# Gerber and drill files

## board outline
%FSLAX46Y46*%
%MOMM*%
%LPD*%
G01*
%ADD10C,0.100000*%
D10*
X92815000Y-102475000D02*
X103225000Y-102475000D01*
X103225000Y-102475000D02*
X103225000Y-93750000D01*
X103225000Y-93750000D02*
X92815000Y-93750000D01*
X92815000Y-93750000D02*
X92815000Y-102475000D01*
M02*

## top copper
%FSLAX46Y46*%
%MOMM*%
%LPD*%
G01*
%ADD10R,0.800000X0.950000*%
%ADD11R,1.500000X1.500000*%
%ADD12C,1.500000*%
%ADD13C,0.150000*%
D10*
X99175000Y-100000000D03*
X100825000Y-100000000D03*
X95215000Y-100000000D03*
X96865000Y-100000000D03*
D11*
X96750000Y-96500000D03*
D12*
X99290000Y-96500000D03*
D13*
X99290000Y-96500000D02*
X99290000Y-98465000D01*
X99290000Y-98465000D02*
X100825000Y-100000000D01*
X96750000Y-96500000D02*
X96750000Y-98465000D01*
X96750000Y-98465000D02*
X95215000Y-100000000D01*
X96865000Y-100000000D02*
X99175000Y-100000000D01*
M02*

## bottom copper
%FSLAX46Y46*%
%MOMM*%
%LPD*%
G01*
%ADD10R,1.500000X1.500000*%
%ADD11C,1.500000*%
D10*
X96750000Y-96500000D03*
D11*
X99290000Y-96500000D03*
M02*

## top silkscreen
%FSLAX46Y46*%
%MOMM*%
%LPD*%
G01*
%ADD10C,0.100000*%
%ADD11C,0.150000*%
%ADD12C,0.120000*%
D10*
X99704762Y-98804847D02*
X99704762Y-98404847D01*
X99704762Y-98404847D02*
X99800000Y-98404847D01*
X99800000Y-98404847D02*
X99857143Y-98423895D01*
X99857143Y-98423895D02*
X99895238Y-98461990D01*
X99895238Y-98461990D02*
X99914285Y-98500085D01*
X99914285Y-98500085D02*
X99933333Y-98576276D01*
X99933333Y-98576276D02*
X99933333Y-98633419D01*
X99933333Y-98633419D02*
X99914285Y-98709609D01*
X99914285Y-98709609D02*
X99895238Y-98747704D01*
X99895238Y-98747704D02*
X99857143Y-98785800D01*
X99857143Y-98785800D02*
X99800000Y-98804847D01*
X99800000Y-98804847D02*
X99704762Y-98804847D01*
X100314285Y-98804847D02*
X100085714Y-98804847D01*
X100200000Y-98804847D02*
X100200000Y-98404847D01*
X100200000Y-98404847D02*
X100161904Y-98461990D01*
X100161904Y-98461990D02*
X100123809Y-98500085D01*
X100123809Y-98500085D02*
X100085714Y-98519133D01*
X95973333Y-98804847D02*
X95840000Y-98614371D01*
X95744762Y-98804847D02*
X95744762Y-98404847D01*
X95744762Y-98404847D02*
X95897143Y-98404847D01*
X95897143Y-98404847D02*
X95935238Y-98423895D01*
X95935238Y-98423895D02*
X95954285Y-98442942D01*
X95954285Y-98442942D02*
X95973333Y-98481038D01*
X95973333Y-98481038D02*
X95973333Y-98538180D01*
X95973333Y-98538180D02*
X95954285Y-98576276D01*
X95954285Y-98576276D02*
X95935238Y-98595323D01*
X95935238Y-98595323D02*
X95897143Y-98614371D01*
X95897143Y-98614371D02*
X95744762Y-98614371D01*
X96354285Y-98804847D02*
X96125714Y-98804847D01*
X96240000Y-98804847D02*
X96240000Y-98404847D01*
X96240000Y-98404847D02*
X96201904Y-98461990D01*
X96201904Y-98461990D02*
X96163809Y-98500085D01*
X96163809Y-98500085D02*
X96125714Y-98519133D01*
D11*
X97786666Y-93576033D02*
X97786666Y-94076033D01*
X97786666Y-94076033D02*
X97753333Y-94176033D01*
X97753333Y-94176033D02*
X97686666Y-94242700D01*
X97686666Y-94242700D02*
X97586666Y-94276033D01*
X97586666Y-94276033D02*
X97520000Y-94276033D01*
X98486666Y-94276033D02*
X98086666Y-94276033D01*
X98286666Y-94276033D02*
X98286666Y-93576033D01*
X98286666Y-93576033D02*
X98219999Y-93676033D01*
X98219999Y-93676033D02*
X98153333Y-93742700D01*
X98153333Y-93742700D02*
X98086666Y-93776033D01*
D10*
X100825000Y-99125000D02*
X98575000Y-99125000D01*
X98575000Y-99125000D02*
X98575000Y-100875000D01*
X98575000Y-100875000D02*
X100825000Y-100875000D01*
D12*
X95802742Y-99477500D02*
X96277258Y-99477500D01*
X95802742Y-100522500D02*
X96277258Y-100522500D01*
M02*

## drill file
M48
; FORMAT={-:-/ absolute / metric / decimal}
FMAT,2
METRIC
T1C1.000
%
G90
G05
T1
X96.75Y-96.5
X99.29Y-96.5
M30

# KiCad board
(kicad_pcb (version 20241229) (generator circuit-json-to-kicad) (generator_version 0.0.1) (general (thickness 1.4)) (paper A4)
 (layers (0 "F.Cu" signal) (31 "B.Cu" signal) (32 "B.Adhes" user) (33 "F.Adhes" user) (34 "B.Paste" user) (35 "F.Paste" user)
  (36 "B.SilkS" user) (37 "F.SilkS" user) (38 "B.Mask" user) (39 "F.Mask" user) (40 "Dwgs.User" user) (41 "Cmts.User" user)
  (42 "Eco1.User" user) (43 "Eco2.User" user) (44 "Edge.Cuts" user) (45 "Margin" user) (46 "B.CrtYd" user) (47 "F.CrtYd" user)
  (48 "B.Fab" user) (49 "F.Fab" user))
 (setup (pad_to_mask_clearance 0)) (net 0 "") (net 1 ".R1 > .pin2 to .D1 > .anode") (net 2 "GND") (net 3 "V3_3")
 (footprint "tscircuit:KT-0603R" (layer F.Cu) (at 100 100 0)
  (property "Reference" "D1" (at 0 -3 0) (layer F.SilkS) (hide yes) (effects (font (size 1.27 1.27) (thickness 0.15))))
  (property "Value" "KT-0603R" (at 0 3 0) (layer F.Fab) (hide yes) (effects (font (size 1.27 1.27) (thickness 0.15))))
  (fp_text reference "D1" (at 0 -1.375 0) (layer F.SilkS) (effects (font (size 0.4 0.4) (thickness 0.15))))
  (fp_line (start 0.825 -0.875) (end -1.425 -0.875) (stroke (width 0.1) (type default)) (layer F.SilkS))
  (fp_line (start -1.425 -0.875) (end -1.425 0.875) (stroke (width 0.1) (type default)) (layer F.SilkS))
  (fp_line (start -1.425 0.875) (end 0.825 0.875) (stroke (width 0.1) (type default)) (layer F.SilkS))
  (pad "1" smd rect (at -0.825 0 0) (size 0.8 0.95) (layers F.Cu F.Paste F.Mask) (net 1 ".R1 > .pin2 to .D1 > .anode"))
  (pad "2" smd rect (at 0.825 0 0) (size 0.8 0.95) (layers F.Cu F.Paste F.Mask) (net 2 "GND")))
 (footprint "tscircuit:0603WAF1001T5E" (layer F.Cu) (at 96.04 100 0)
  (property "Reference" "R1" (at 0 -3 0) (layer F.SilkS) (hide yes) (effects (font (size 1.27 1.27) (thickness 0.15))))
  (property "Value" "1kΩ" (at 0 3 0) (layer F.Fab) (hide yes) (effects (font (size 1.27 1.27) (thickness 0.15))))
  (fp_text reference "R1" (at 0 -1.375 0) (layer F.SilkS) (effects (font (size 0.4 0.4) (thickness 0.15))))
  (fp_line (start -0.2372580000000002 -0.5225) (end 0.2372580000000002 -0.5225) (stroke (width 0.12) (type default)) (layer F.SilkS))
  (fp_line (start -0.2372580000000002 0.5225) (end 0.2372580000000002 0.5225) (stroke (width 0.12) (type default)) (layer F.SilkS))
  (pad "1" smd rect (at -0.8249999999999997 0 0) (size 0.8 0.95) (layers F.Cu F.Paste F.Mask) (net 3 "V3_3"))
  (pad "2" smd rect (at 0.8249999999999997 0 0) (size 0.8 0.95) (layers F.Cu F.Paste F.Mask) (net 1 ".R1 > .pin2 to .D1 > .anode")))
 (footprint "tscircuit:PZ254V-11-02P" (layer F.Cu) (at 98.02 96.5 0)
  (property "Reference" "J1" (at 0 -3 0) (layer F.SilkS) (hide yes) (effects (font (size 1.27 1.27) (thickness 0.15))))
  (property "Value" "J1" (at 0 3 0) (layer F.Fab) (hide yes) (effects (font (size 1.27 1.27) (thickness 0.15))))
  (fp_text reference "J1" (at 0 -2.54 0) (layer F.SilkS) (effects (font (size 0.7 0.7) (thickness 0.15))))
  (pad "1" thru_hole rect (at -1.27 0 0) (size 1.5 1.5) (drill 1) (layers *.Cu *.Mask) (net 3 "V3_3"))
  (pad "2" thru_hole circle (at 1.27 0 0) (size 1.5 1.5) (drill 1) (layers *.Cu *.Mask) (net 2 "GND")))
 (segment (start 99.29 96.5) (end 99.29 98.465) (width 0.15) (layer F.Cu) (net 2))
 (segment (start 99.29 98.465) (end 100.825 100) (width 0.15) (layer F.Cu) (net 2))
 (segment (start 96.75 96.5) (end 96.75 98.465) (width 0.15) (layer F.Cu) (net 3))
 (segment (start 96.75 98.465) (end 95.215 100) (width 0.15) (layer F.Cu) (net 3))
 (segment (start 96.865 100) (end 99.175 100) (width 0.15) (layer F.Cu) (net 1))
 (gr_line (start 92.815 102.475) (end 103.225 102.475) (width 0.1) (layer Edge.Cuts))
 (gr_line (start 103.225 102.475) (end 103.225 93.75) (width 0.1) (layer Edge.Cuts))
 (gr_line (start 103.225 93.75) (end 92.815 93.75) (width 0.1) (layer Edge.Cuts))
 (gr_line (start 92.815 93.75) (end 92.815 102.475) (width 0.1) (layer Edge.Cuts)))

